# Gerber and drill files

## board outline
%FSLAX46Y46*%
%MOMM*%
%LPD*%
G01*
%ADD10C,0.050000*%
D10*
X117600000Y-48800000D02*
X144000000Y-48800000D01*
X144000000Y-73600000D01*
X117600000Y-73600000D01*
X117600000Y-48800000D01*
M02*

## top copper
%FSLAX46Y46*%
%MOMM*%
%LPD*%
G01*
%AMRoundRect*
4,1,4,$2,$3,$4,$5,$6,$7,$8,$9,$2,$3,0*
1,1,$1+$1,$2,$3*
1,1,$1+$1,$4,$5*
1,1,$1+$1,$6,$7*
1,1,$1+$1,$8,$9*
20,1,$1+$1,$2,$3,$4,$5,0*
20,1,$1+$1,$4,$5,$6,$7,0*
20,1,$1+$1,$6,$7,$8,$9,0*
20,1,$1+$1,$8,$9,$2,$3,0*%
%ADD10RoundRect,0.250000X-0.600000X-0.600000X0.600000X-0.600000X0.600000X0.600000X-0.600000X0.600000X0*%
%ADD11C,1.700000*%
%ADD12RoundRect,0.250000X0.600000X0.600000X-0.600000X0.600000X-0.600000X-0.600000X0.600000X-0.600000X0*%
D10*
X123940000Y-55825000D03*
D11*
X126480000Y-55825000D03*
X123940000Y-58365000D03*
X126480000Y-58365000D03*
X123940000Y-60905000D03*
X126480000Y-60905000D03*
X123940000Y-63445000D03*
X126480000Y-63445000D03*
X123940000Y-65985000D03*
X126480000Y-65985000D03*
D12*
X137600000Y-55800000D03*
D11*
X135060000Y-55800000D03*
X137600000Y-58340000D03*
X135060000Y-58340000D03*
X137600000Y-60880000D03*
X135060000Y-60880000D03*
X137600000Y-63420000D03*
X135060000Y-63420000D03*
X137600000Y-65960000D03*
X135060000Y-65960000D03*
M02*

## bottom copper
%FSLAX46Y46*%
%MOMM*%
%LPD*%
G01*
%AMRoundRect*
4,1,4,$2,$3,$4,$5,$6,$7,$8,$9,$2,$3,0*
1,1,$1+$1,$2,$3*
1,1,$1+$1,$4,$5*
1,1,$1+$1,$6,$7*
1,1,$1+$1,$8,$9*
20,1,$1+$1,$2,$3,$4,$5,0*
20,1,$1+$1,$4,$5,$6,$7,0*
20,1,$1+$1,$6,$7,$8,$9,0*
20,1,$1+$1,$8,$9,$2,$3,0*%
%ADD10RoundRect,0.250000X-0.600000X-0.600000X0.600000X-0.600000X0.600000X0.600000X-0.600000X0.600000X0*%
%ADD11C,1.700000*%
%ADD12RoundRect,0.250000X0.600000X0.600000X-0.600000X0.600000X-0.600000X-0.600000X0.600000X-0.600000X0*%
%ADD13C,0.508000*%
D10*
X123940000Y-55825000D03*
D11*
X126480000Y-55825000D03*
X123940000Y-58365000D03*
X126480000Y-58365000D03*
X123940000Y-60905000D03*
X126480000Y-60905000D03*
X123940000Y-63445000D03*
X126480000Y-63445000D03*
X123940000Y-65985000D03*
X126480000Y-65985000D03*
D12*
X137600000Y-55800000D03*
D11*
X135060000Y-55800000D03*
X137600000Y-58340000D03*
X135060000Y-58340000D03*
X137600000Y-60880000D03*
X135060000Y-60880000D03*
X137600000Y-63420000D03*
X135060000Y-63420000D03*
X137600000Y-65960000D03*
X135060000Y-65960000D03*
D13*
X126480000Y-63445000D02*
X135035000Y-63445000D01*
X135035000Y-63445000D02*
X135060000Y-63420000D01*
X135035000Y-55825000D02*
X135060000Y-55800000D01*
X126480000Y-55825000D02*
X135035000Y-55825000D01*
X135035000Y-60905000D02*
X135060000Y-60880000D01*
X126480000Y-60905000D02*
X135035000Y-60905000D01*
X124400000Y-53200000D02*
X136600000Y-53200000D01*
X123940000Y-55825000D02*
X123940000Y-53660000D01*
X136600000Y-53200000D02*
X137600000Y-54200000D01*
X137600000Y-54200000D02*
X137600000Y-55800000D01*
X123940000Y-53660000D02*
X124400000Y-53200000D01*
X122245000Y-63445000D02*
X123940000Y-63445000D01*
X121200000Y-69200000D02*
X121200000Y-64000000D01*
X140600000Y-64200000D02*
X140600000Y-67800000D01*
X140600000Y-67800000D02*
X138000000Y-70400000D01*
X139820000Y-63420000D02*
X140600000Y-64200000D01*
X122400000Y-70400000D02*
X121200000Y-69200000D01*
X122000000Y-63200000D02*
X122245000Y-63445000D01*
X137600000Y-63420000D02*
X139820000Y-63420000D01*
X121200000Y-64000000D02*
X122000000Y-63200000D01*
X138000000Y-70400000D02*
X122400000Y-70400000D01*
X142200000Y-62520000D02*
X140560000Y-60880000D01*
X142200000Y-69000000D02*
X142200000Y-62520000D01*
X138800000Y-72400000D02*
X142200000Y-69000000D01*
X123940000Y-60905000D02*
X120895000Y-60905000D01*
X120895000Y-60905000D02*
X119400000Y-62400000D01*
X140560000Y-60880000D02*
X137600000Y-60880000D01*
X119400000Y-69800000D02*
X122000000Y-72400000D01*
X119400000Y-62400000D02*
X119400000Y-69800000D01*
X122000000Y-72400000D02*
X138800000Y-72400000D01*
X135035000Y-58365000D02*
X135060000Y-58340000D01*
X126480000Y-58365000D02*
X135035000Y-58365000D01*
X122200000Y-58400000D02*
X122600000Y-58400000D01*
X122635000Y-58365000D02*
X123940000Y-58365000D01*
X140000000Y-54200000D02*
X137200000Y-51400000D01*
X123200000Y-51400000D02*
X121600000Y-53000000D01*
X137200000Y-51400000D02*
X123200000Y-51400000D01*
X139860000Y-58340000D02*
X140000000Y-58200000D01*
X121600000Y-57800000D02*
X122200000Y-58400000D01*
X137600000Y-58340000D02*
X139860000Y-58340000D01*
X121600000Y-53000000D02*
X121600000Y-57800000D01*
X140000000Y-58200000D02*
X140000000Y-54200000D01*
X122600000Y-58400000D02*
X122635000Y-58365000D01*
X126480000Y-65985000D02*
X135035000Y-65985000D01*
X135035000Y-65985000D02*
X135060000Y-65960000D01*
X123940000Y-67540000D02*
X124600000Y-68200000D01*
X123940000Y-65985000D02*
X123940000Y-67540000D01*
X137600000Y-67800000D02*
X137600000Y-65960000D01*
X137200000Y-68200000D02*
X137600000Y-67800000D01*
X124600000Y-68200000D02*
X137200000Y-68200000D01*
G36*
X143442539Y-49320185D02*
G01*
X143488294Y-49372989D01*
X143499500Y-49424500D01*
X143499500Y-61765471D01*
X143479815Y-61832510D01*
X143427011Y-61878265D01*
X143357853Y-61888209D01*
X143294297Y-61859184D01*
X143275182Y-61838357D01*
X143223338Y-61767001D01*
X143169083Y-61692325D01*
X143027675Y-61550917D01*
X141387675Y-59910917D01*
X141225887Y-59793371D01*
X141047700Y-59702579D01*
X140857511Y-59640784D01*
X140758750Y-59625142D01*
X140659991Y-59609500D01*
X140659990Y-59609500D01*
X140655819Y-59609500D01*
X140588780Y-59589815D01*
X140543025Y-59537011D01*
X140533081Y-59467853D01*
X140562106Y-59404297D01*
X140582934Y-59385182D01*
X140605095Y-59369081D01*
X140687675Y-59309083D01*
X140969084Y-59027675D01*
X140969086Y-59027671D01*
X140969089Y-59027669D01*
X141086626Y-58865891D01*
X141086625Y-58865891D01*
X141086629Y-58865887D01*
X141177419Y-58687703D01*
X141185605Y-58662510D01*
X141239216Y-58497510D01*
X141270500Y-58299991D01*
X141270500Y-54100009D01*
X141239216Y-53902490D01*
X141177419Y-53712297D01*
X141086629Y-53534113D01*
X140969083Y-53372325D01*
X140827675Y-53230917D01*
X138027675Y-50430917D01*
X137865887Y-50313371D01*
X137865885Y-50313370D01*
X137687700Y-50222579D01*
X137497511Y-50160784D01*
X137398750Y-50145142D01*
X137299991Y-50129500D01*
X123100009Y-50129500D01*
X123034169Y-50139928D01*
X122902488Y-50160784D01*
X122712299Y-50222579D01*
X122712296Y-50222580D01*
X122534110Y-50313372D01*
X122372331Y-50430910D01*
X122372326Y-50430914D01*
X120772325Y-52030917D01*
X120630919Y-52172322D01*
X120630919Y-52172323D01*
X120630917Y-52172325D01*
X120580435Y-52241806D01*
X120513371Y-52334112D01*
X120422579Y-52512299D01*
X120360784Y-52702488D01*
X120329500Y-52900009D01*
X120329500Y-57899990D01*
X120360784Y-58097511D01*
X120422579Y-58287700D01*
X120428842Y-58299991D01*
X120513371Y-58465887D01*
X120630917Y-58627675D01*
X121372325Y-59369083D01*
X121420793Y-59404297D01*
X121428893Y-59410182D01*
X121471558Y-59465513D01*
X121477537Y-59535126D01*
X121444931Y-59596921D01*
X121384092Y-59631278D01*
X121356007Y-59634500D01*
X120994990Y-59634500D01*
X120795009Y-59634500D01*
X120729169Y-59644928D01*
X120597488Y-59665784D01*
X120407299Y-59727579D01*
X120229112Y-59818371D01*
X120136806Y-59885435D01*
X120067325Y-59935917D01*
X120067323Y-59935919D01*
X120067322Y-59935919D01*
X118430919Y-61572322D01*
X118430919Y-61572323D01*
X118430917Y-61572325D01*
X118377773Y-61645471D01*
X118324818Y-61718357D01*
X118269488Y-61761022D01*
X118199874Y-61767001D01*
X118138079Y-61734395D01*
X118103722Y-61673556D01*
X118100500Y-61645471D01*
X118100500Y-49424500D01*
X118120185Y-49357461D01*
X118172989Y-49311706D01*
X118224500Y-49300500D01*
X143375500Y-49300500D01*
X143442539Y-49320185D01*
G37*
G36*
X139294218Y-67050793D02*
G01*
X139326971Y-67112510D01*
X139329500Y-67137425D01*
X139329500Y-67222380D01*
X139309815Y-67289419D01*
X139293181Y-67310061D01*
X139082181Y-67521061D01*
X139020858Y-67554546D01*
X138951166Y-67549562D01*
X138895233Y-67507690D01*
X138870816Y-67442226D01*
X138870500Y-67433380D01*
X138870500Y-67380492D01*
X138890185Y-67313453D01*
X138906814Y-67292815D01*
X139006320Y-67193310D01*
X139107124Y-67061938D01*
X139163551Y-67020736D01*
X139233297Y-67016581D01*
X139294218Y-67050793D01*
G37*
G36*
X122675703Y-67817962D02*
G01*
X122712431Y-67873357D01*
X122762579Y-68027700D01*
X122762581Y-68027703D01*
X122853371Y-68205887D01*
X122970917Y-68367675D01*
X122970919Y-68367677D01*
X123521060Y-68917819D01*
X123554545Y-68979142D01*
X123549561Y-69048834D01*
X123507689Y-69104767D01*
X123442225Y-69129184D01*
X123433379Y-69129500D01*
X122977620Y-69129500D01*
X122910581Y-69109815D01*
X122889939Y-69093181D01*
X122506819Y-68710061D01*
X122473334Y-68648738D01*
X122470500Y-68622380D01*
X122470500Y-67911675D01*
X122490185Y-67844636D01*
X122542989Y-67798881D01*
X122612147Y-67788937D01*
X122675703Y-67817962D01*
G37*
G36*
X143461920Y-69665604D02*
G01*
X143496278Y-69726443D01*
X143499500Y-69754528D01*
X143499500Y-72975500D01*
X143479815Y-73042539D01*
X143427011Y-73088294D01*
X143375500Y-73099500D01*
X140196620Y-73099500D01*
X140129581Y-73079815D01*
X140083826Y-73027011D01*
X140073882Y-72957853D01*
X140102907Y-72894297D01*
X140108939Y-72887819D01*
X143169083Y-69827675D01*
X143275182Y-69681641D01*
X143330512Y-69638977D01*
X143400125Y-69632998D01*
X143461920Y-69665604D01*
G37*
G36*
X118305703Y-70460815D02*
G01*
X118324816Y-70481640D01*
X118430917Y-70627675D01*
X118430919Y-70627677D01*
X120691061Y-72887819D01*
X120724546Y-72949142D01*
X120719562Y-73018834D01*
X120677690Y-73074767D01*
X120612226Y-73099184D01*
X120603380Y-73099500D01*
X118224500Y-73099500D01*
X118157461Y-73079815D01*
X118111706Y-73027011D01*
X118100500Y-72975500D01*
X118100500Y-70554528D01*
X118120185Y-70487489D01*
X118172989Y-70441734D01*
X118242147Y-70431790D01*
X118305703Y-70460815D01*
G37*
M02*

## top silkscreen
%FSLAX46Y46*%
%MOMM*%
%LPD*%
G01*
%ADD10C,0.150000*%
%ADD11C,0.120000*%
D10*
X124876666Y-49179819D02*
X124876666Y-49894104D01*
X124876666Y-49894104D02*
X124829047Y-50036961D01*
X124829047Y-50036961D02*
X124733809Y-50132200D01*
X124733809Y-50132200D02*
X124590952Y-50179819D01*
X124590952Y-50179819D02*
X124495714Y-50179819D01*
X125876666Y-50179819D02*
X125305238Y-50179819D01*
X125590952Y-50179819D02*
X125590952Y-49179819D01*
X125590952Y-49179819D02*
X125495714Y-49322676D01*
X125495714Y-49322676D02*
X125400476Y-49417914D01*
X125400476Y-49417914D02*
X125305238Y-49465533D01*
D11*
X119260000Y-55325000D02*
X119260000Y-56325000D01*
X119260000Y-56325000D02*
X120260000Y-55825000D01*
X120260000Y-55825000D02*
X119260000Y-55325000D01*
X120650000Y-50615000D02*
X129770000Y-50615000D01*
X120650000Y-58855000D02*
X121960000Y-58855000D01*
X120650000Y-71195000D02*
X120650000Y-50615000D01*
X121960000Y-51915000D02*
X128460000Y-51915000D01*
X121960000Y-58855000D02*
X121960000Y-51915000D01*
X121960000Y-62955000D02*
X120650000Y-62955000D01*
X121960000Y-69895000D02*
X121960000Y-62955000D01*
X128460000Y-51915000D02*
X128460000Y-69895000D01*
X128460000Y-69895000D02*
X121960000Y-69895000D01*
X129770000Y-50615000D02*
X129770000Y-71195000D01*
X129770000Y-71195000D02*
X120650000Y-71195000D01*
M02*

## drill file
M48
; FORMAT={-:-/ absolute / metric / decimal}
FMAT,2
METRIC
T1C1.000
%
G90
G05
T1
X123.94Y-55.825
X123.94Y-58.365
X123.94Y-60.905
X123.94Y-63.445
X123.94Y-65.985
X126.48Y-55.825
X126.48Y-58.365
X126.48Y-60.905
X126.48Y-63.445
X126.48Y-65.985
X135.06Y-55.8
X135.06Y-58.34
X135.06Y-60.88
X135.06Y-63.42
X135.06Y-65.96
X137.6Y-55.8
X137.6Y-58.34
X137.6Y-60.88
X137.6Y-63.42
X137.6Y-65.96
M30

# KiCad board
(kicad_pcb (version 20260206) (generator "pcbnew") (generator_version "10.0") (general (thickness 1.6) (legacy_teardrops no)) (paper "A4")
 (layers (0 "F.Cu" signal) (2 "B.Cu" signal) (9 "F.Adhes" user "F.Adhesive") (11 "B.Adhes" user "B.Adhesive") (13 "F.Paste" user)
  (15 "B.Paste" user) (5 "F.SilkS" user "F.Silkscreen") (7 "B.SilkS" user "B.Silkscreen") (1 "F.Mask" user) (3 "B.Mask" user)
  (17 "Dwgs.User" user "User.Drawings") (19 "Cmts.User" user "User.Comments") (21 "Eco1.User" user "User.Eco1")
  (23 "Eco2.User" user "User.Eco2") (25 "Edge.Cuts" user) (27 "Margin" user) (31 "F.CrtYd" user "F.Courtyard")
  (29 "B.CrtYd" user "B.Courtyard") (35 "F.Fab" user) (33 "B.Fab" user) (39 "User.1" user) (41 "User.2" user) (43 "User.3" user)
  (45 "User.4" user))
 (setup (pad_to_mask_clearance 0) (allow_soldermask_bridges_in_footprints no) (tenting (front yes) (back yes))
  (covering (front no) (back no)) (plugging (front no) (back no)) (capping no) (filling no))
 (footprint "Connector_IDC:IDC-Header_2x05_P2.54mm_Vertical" (layer "F.Cu") (at 123.94 55.825)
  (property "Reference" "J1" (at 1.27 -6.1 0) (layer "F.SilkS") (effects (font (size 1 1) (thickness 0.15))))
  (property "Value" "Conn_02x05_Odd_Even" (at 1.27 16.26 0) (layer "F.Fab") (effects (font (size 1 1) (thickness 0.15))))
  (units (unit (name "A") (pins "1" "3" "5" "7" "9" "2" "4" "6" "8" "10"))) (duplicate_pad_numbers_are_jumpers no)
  (fp_line (start -4.68 -0.5) (end -4.68 0.5) (stroke (width 0.12) (type solid)) (layer "F.SilkS"))
  (fp_line (start -4.68 0.5) (end -3.68 0) (stroke (width 0.12) (type solid)) (layer "F.SilkS"))
  (fp_line (start -3.68 0) (end -4.68 -0.5) (stroke (width 0.12) (type solid)) (layer "F.SilkS"))
  (fp_line (start -3.29 -5.21) (end 5.83 -5.21) (stroke (width 0.12) (type solid)) (layer "F.SilkS"))
  (fp_line (start -3.29 3.03) (end -1.98 3.03) (stroke (width 0.12) (type solid)) (layer "F.SilkS"))
  (fp_line (start -3.29 15.37) (end -3.29 -5.21) (stroke (width 0.12) (type solid)) (layer "F.SilkS"))
  (fp_line (start -1.98 -3.91) (end 4.52 -3.91) (stroke (width 0.12) (type solid)) (layer "F.SilkS"))
  (fp_line (start -1.98 3.03) (end -1.98 -3.91) (stroke (width 0.12) (type solid)) (layer "F.SilkS"))
  (fp_line (start -1.98 7.13) (end -3.29 7.13) (stroke (width 0.12) (type solid)) (layer "F.SilkS"))
  (fp_line (start -1.98 14.07) (end -1.98 7.13) (stroke (width 0.12) (type solid)) (layer "F.SilkS"))
  (fp_line (start 4.52 -3.91) (end 4.52 14.07) (stroke (width 0.12) (type solid)) (layer "F.SilkS"))
  (fp_line (start 4.52 14.07) (end -1.98 14.07) (stroke (width 0.12) (type solid)) (layer "F.SilkS"))
  (fp_line (start 5.83 -5.21) (end 5.83 15.37) (stroke (width 0.12) (type solid)) (layer "F.SilkS"))
  (fp_line (start 5.83 15.37) (end -3.29 15.37) (stroke (width 0.12) (type solid)) (layer "F.SilkS"))
  (pad "1" thru_hole roundrect (at 0 0) (size 1.7 1.7) (drill 1) (layers "*.Cu" "*.Mask") (remove_unused_layers no)
   (roundrect_rratio 0.147059) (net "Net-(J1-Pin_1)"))
  (pad "2" thru_hole circle (at 2.54 0) (size 1.7 1.7) (drill 1) (layers "*.Cu" "*.Mask") (remove_unused_layers no) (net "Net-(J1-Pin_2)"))
  (pad "3" thru_hole circle (at 0 2.54) (size 1.7 1.7) (drill 1) (layers "*.Cu" "*.Mask") (remove_unused_layers no) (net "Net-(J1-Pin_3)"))
  (pad "4" thru_hole circle (at 2.54 2.54) (size 1.7 1.7) (drill 1) (layers "*.Cu" "*.Mask") (remove_unused_layers no)
   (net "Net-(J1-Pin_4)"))
  (pad "5" thru_hole circle (at 0 5.08) (size 1.7 1.7) (drill 1) (layers "*.Cu" "*.Mask") (remove_unused_layers no) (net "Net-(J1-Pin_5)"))
  (pad "6" thru_hole circle (at 2.54 5.08) (size 1.7 1.7) (drill 1) (layers "*.Cu" "*.Mask") (remove_unused_layers no)
   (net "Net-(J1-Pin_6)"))
  (pad "7" thru_hole circle (at 0 7.62) (size 1.7 1.7) (drill 1) (layers "*.Cu" "*.Mask") (remove_unused_layers no) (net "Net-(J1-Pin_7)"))
  (pad "8" thru_hole circle (at 2.54 7.62) (size 1.7 1.7) (drill 1) (layers "*.Cu" "*.Mask") (remove_unused_layers no)
   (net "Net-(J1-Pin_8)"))
  (pad "9" thru_hole circle (at 0 10.16) (size 1.7 1.7) (drill 1) (layers "*.Cu" "*.Mask") (remove_unused_layers no) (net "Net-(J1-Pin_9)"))
  (pad "10" thru_hole circle (at 2.54 10.16) (size 1.7 1.7) (drill 1) (layers "*.Cu" "*.Mask") (remove_unused_layers no)
   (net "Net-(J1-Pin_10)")))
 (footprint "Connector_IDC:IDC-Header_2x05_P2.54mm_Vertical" (layer "B.Cu") (at 137.6 55.8 180)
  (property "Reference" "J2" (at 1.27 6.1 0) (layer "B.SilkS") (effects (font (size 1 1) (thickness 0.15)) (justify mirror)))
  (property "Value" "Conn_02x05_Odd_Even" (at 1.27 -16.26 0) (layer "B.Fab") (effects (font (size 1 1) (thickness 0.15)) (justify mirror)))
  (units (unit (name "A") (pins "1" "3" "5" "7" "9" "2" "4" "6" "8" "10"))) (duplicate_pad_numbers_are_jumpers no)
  (pad "1" thru_hole roundrect (at 0 0 180) (size 1.7 1.7) (drill 1) (layers "*.Cu" "*.Mask") (remove_unused_layers no)
   (roundrect_rratio 0.147059) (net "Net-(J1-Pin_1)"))
  (pad "2" thru_hole circle (at 2.54 0 180) (size 1.7 1.7) (drill 1) (layers "*.Cu" "*.Mask") (remove_unused_layers no)
   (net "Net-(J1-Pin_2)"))
  (pad "3" thru_hole circle (at 0 -2.54 180) (size 1.7 1.7) (drill 1) (layers "*.Cu" "*.Mask") (remove_unused_layers no)
   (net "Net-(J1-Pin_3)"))
  (pad "4" thru_hole circle (at 2.54 -2.54 180) (size 1.7 1.7) (drill 1) (layers "*.Cu" "*.Mask") (remove_unused_layers no)
   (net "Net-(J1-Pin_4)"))
  (pad "5" thru_hole circle (at 0 -5.08 180) (size 1.7 1.7) (drill 1) (layers "*.Cu" "*.Mask") (remove_unused_layers no)
   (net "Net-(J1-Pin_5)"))
  (pad "6" thru_hole circle (at 2.54 -5.08 180) (size 1.7 1.7) (drill 1) (layers "*.Cu" "*.Mask") (remove_unused_layers no)
   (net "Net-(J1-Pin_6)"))
  (pad "7" thru_hole circle (at 0 -7.62 180) (size 1.7 1.7) (drill 1) (layers "*.Cu" "*.Mask") (remove_unused_layers no)
   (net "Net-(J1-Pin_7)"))
  (pad "8" thru_hole circle (at 2.54 -7.62 180) (size 1.7 1.7) (drill 1) (layers "*.Cu" "*.Mask") (remove_unused_layers no)
   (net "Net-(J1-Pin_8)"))
  (pad "9" thru_hole circle (at 0 -10.16 180) (size 1.7 1.7) (drill 1) (layers "*.Cu" "*.Mask") (remove_unused_layers no)
   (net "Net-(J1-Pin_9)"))
  (pad "10" thru_hole circle (at 2.54 -10.16 180) (size 1.7 1.7) (drill 1) (layers "*.Cu" "*.Mask") (remove_unused_layers no)
   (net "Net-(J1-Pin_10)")))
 (gr_rect (start 117.6 48.8) (end 144 73.6) (stroke (width 0.05) (type default)) (fill no) (layer "Edge.Cuts"))
 (segment (start 126.48 63.445) (end 135.035 63.445) (width 0.508) (layer "B.Cu") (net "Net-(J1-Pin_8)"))
 (segment (start 135.035 63.445) (end 135.06 63.42) (width 0.508) (layer "B.Cu") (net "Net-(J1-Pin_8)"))
 (segment (start 135.035 55.825) (end 135.06 55.8) (width 0.508) (layer "B.Cu") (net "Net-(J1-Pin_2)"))
 (segment (start 126.48 55.825) (end 135.035 55.825) (width 0.508) (layer "B.Cu") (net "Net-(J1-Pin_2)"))
 (segment (start 135.035 60.905) (end 135.06 60.88) (width 0.508) (layer "B.Cu") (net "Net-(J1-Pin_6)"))
 (segment (start 126.48 60.905) (end 135.035 60.905) (width 0.508) (layer "B.Cu") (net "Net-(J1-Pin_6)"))
 (segment (start 124.4 53.2) (end 136.6 53.2) (width 0.508) (layer "B.Cu") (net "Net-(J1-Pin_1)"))
 (segment (start 123.94 55.825) (end 123.94 53.66) (width 0.508) (layer "B.Cu") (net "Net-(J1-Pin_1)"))
 (segment (start 136.6 53.2) (end 137.6 54.2) (width 0.508) (layer "B.Cu") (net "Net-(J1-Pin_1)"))
 (segment (start 137.6 54.2) (end 137.6 55.8) (width 0.508) (layer "B.Cu") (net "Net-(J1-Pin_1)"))
 (segment (start 123.94 53.66) (end 124.4 53.2) (width 0.508) (layer "B.Cu") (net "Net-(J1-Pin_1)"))
 (segment (start 122.245 63.445) (end 123.94 63.445) (width 0.508) (layer "B.Cu") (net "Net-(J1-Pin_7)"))
 (segment (start 121.2 69.2) (end 121.2 64) (width 0.508) (layer "B.Cu") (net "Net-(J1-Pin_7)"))
 (segment (start 140.6 64.2) (end 140.6 67.8) (width 0.508) (layer "B.Cu") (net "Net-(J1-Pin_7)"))
 (segment (start 140.6 67.8) (end 138 70.4) (width 0.508) (layer "B.Cu") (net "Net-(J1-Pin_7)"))
 (segment (start 139.82 63.42) (end 140.6 64.2) (width 0.508) (layer "B.Cu") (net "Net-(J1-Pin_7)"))
 (segment (start 122.4 70.4) (end 121.2 69.2) (width 0.508) (layer "B.Cu") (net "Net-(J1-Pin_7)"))
 (segment (start 122 63.2) (end 122.245 63.445) (width 0.508) (layer "B.Cu") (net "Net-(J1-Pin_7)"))
 (segment (start 137.6 63.42) (end 139.82 63.42) (width 0.508) (layer "B.Cu") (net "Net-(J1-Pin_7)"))
 (segment (start 121.2 64) (end 122 63.2) (width 0.508) (layer "B.Cu") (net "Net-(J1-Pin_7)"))
 (segment (start 138 70.4) (end 122.4 70.4) (width 0.508) (layer "B.Cu") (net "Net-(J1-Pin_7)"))
 (segment (start 142.2 62.52) (end 140.56 60.88) (width 0.508) (layer "B.Cu") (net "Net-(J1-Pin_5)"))
 (segment (start 142.2 69) (end 142.2 62.52) (width 0.508) (layer "B.Cu") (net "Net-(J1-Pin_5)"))
 (segment (start 138.8 72.4) (end 142.2 69) (width 0.508) (layer "B.Cu") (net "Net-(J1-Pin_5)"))
 (segment (start 123.94 60.905) (end 120.895 60.905) (width 0.508) (layer "B.Cu") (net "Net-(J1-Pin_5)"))
 (segment (start 120.895 60.905) (end 119.4 62.4) (width 0.508) (layer "B.Cu") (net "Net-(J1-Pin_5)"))
 (segment (start 140.56 60.88) (end 137.6 60.88) (width 0.508) (layer "B.Cu") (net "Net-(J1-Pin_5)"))
 (segment (start 119.4 69.8) (end 122 72.4) (width 0.508) (layer "B.Cu") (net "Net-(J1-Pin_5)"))
 (segment (start 119.4 62.4) (end 119.4 69.8) (width 0.508) (layer "B.Cu") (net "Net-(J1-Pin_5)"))
 (segment (start 122 72.4) (end 138.8 72.4) (width 0.508) (layer "B.Cu") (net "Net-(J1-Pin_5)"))
 (segment (start 135.035 58.365) (end 135.06 58.34) (width 0.508) (layer "B.Cu") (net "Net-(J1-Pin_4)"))
 (segment (start 126.48 58.365) (end 135.035 58.365) (width 0.508) (layer "B.Cu") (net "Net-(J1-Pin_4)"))
 (segment (start 122.2 58.4) (end 122.6 58.4) (width 0.508) (layer "B.Cu") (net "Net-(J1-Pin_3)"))
 (segment (start 122.635 58.365) (end 123.94 58.365) (width 0.508) (layer "B.Cu") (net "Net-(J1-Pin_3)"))
 (segment (start 140 54.2) (end 137.2 51.4) (width 0.508) (layer "B.Cu") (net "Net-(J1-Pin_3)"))
 (segment (start 123.2 51.4) (end 121.6 53) (width 0.508) (layer "B.Cu") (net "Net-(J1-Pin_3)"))
 (segment (start 137.2 51.4) (end 123.2 51.4) (width 0.508) (layer "B.Cu") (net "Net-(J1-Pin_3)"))
 (segment (start 139.86 58.34) (end 140 58.2) (width 0.508) (layer "B.Cu") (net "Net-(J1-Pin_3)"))
 (segment (start 121.6 57.8) (end 122.2 58.4) (width 0.508) (layer "B.Cu") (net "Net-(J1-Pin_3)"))
 (segment (start 137.6 58.34) (end 139.86 58.34) (width 0.508) (layer "B.Cu") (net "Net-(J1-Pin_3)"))
 (segment (start 121.6 53) (end 121.6 57.8) (width 0.508) (layer "B.Cu") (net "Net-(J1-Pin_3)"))
 (segment (start 140 58.2) (end 140 54.2) (width 0.508) (layer "B.Cu") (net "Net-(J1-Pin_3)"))
 (segment (start 122.6 58.4) (end 122.635 58.365) (width 0.508) (layer "B.Cu") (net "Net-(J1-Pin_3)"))
 (segment (start 126.48 65.985) (end 135.035 65.985) (width 0.508) (layer "B.Cu") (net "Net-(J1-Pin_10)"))
 (segment (start 135.035 65.985) (end 135.06 65.96) (width 0.508) (layer "B.Cu") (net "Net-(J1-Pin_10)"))
 (segment (start 123.94 67.54) (end 124.6 68.2) (width 0.508) (layer "B.Cu") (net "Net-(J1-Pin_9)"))
 (segment (start 123.94 65.985) (end 123.94 67.54) (width 0.508) (layer "B.Cu") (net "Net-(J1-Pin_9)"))
 (segment (start 137.6 67.8) (end 137.6 65.96) (width 0.508) (layer "B.Cu") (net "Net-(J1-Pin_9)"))
 (segment (start 137.2 68.2) (end 137.6 67.8) (width 0.508) (layer "B.Cu") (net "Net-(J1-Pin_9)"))
 (segment (start 124.6 68.2) (end 137.2 68.2) (width 0.508) (layer "B.Cu") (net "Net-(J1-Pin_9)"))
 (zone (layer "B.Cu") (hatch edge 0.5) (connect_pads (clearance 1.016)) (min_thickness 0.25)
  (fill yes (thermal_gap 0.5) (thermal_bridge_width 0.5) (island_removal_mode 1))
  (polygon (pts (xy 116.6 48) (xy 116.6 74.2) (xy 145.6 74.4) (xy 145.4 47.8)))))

